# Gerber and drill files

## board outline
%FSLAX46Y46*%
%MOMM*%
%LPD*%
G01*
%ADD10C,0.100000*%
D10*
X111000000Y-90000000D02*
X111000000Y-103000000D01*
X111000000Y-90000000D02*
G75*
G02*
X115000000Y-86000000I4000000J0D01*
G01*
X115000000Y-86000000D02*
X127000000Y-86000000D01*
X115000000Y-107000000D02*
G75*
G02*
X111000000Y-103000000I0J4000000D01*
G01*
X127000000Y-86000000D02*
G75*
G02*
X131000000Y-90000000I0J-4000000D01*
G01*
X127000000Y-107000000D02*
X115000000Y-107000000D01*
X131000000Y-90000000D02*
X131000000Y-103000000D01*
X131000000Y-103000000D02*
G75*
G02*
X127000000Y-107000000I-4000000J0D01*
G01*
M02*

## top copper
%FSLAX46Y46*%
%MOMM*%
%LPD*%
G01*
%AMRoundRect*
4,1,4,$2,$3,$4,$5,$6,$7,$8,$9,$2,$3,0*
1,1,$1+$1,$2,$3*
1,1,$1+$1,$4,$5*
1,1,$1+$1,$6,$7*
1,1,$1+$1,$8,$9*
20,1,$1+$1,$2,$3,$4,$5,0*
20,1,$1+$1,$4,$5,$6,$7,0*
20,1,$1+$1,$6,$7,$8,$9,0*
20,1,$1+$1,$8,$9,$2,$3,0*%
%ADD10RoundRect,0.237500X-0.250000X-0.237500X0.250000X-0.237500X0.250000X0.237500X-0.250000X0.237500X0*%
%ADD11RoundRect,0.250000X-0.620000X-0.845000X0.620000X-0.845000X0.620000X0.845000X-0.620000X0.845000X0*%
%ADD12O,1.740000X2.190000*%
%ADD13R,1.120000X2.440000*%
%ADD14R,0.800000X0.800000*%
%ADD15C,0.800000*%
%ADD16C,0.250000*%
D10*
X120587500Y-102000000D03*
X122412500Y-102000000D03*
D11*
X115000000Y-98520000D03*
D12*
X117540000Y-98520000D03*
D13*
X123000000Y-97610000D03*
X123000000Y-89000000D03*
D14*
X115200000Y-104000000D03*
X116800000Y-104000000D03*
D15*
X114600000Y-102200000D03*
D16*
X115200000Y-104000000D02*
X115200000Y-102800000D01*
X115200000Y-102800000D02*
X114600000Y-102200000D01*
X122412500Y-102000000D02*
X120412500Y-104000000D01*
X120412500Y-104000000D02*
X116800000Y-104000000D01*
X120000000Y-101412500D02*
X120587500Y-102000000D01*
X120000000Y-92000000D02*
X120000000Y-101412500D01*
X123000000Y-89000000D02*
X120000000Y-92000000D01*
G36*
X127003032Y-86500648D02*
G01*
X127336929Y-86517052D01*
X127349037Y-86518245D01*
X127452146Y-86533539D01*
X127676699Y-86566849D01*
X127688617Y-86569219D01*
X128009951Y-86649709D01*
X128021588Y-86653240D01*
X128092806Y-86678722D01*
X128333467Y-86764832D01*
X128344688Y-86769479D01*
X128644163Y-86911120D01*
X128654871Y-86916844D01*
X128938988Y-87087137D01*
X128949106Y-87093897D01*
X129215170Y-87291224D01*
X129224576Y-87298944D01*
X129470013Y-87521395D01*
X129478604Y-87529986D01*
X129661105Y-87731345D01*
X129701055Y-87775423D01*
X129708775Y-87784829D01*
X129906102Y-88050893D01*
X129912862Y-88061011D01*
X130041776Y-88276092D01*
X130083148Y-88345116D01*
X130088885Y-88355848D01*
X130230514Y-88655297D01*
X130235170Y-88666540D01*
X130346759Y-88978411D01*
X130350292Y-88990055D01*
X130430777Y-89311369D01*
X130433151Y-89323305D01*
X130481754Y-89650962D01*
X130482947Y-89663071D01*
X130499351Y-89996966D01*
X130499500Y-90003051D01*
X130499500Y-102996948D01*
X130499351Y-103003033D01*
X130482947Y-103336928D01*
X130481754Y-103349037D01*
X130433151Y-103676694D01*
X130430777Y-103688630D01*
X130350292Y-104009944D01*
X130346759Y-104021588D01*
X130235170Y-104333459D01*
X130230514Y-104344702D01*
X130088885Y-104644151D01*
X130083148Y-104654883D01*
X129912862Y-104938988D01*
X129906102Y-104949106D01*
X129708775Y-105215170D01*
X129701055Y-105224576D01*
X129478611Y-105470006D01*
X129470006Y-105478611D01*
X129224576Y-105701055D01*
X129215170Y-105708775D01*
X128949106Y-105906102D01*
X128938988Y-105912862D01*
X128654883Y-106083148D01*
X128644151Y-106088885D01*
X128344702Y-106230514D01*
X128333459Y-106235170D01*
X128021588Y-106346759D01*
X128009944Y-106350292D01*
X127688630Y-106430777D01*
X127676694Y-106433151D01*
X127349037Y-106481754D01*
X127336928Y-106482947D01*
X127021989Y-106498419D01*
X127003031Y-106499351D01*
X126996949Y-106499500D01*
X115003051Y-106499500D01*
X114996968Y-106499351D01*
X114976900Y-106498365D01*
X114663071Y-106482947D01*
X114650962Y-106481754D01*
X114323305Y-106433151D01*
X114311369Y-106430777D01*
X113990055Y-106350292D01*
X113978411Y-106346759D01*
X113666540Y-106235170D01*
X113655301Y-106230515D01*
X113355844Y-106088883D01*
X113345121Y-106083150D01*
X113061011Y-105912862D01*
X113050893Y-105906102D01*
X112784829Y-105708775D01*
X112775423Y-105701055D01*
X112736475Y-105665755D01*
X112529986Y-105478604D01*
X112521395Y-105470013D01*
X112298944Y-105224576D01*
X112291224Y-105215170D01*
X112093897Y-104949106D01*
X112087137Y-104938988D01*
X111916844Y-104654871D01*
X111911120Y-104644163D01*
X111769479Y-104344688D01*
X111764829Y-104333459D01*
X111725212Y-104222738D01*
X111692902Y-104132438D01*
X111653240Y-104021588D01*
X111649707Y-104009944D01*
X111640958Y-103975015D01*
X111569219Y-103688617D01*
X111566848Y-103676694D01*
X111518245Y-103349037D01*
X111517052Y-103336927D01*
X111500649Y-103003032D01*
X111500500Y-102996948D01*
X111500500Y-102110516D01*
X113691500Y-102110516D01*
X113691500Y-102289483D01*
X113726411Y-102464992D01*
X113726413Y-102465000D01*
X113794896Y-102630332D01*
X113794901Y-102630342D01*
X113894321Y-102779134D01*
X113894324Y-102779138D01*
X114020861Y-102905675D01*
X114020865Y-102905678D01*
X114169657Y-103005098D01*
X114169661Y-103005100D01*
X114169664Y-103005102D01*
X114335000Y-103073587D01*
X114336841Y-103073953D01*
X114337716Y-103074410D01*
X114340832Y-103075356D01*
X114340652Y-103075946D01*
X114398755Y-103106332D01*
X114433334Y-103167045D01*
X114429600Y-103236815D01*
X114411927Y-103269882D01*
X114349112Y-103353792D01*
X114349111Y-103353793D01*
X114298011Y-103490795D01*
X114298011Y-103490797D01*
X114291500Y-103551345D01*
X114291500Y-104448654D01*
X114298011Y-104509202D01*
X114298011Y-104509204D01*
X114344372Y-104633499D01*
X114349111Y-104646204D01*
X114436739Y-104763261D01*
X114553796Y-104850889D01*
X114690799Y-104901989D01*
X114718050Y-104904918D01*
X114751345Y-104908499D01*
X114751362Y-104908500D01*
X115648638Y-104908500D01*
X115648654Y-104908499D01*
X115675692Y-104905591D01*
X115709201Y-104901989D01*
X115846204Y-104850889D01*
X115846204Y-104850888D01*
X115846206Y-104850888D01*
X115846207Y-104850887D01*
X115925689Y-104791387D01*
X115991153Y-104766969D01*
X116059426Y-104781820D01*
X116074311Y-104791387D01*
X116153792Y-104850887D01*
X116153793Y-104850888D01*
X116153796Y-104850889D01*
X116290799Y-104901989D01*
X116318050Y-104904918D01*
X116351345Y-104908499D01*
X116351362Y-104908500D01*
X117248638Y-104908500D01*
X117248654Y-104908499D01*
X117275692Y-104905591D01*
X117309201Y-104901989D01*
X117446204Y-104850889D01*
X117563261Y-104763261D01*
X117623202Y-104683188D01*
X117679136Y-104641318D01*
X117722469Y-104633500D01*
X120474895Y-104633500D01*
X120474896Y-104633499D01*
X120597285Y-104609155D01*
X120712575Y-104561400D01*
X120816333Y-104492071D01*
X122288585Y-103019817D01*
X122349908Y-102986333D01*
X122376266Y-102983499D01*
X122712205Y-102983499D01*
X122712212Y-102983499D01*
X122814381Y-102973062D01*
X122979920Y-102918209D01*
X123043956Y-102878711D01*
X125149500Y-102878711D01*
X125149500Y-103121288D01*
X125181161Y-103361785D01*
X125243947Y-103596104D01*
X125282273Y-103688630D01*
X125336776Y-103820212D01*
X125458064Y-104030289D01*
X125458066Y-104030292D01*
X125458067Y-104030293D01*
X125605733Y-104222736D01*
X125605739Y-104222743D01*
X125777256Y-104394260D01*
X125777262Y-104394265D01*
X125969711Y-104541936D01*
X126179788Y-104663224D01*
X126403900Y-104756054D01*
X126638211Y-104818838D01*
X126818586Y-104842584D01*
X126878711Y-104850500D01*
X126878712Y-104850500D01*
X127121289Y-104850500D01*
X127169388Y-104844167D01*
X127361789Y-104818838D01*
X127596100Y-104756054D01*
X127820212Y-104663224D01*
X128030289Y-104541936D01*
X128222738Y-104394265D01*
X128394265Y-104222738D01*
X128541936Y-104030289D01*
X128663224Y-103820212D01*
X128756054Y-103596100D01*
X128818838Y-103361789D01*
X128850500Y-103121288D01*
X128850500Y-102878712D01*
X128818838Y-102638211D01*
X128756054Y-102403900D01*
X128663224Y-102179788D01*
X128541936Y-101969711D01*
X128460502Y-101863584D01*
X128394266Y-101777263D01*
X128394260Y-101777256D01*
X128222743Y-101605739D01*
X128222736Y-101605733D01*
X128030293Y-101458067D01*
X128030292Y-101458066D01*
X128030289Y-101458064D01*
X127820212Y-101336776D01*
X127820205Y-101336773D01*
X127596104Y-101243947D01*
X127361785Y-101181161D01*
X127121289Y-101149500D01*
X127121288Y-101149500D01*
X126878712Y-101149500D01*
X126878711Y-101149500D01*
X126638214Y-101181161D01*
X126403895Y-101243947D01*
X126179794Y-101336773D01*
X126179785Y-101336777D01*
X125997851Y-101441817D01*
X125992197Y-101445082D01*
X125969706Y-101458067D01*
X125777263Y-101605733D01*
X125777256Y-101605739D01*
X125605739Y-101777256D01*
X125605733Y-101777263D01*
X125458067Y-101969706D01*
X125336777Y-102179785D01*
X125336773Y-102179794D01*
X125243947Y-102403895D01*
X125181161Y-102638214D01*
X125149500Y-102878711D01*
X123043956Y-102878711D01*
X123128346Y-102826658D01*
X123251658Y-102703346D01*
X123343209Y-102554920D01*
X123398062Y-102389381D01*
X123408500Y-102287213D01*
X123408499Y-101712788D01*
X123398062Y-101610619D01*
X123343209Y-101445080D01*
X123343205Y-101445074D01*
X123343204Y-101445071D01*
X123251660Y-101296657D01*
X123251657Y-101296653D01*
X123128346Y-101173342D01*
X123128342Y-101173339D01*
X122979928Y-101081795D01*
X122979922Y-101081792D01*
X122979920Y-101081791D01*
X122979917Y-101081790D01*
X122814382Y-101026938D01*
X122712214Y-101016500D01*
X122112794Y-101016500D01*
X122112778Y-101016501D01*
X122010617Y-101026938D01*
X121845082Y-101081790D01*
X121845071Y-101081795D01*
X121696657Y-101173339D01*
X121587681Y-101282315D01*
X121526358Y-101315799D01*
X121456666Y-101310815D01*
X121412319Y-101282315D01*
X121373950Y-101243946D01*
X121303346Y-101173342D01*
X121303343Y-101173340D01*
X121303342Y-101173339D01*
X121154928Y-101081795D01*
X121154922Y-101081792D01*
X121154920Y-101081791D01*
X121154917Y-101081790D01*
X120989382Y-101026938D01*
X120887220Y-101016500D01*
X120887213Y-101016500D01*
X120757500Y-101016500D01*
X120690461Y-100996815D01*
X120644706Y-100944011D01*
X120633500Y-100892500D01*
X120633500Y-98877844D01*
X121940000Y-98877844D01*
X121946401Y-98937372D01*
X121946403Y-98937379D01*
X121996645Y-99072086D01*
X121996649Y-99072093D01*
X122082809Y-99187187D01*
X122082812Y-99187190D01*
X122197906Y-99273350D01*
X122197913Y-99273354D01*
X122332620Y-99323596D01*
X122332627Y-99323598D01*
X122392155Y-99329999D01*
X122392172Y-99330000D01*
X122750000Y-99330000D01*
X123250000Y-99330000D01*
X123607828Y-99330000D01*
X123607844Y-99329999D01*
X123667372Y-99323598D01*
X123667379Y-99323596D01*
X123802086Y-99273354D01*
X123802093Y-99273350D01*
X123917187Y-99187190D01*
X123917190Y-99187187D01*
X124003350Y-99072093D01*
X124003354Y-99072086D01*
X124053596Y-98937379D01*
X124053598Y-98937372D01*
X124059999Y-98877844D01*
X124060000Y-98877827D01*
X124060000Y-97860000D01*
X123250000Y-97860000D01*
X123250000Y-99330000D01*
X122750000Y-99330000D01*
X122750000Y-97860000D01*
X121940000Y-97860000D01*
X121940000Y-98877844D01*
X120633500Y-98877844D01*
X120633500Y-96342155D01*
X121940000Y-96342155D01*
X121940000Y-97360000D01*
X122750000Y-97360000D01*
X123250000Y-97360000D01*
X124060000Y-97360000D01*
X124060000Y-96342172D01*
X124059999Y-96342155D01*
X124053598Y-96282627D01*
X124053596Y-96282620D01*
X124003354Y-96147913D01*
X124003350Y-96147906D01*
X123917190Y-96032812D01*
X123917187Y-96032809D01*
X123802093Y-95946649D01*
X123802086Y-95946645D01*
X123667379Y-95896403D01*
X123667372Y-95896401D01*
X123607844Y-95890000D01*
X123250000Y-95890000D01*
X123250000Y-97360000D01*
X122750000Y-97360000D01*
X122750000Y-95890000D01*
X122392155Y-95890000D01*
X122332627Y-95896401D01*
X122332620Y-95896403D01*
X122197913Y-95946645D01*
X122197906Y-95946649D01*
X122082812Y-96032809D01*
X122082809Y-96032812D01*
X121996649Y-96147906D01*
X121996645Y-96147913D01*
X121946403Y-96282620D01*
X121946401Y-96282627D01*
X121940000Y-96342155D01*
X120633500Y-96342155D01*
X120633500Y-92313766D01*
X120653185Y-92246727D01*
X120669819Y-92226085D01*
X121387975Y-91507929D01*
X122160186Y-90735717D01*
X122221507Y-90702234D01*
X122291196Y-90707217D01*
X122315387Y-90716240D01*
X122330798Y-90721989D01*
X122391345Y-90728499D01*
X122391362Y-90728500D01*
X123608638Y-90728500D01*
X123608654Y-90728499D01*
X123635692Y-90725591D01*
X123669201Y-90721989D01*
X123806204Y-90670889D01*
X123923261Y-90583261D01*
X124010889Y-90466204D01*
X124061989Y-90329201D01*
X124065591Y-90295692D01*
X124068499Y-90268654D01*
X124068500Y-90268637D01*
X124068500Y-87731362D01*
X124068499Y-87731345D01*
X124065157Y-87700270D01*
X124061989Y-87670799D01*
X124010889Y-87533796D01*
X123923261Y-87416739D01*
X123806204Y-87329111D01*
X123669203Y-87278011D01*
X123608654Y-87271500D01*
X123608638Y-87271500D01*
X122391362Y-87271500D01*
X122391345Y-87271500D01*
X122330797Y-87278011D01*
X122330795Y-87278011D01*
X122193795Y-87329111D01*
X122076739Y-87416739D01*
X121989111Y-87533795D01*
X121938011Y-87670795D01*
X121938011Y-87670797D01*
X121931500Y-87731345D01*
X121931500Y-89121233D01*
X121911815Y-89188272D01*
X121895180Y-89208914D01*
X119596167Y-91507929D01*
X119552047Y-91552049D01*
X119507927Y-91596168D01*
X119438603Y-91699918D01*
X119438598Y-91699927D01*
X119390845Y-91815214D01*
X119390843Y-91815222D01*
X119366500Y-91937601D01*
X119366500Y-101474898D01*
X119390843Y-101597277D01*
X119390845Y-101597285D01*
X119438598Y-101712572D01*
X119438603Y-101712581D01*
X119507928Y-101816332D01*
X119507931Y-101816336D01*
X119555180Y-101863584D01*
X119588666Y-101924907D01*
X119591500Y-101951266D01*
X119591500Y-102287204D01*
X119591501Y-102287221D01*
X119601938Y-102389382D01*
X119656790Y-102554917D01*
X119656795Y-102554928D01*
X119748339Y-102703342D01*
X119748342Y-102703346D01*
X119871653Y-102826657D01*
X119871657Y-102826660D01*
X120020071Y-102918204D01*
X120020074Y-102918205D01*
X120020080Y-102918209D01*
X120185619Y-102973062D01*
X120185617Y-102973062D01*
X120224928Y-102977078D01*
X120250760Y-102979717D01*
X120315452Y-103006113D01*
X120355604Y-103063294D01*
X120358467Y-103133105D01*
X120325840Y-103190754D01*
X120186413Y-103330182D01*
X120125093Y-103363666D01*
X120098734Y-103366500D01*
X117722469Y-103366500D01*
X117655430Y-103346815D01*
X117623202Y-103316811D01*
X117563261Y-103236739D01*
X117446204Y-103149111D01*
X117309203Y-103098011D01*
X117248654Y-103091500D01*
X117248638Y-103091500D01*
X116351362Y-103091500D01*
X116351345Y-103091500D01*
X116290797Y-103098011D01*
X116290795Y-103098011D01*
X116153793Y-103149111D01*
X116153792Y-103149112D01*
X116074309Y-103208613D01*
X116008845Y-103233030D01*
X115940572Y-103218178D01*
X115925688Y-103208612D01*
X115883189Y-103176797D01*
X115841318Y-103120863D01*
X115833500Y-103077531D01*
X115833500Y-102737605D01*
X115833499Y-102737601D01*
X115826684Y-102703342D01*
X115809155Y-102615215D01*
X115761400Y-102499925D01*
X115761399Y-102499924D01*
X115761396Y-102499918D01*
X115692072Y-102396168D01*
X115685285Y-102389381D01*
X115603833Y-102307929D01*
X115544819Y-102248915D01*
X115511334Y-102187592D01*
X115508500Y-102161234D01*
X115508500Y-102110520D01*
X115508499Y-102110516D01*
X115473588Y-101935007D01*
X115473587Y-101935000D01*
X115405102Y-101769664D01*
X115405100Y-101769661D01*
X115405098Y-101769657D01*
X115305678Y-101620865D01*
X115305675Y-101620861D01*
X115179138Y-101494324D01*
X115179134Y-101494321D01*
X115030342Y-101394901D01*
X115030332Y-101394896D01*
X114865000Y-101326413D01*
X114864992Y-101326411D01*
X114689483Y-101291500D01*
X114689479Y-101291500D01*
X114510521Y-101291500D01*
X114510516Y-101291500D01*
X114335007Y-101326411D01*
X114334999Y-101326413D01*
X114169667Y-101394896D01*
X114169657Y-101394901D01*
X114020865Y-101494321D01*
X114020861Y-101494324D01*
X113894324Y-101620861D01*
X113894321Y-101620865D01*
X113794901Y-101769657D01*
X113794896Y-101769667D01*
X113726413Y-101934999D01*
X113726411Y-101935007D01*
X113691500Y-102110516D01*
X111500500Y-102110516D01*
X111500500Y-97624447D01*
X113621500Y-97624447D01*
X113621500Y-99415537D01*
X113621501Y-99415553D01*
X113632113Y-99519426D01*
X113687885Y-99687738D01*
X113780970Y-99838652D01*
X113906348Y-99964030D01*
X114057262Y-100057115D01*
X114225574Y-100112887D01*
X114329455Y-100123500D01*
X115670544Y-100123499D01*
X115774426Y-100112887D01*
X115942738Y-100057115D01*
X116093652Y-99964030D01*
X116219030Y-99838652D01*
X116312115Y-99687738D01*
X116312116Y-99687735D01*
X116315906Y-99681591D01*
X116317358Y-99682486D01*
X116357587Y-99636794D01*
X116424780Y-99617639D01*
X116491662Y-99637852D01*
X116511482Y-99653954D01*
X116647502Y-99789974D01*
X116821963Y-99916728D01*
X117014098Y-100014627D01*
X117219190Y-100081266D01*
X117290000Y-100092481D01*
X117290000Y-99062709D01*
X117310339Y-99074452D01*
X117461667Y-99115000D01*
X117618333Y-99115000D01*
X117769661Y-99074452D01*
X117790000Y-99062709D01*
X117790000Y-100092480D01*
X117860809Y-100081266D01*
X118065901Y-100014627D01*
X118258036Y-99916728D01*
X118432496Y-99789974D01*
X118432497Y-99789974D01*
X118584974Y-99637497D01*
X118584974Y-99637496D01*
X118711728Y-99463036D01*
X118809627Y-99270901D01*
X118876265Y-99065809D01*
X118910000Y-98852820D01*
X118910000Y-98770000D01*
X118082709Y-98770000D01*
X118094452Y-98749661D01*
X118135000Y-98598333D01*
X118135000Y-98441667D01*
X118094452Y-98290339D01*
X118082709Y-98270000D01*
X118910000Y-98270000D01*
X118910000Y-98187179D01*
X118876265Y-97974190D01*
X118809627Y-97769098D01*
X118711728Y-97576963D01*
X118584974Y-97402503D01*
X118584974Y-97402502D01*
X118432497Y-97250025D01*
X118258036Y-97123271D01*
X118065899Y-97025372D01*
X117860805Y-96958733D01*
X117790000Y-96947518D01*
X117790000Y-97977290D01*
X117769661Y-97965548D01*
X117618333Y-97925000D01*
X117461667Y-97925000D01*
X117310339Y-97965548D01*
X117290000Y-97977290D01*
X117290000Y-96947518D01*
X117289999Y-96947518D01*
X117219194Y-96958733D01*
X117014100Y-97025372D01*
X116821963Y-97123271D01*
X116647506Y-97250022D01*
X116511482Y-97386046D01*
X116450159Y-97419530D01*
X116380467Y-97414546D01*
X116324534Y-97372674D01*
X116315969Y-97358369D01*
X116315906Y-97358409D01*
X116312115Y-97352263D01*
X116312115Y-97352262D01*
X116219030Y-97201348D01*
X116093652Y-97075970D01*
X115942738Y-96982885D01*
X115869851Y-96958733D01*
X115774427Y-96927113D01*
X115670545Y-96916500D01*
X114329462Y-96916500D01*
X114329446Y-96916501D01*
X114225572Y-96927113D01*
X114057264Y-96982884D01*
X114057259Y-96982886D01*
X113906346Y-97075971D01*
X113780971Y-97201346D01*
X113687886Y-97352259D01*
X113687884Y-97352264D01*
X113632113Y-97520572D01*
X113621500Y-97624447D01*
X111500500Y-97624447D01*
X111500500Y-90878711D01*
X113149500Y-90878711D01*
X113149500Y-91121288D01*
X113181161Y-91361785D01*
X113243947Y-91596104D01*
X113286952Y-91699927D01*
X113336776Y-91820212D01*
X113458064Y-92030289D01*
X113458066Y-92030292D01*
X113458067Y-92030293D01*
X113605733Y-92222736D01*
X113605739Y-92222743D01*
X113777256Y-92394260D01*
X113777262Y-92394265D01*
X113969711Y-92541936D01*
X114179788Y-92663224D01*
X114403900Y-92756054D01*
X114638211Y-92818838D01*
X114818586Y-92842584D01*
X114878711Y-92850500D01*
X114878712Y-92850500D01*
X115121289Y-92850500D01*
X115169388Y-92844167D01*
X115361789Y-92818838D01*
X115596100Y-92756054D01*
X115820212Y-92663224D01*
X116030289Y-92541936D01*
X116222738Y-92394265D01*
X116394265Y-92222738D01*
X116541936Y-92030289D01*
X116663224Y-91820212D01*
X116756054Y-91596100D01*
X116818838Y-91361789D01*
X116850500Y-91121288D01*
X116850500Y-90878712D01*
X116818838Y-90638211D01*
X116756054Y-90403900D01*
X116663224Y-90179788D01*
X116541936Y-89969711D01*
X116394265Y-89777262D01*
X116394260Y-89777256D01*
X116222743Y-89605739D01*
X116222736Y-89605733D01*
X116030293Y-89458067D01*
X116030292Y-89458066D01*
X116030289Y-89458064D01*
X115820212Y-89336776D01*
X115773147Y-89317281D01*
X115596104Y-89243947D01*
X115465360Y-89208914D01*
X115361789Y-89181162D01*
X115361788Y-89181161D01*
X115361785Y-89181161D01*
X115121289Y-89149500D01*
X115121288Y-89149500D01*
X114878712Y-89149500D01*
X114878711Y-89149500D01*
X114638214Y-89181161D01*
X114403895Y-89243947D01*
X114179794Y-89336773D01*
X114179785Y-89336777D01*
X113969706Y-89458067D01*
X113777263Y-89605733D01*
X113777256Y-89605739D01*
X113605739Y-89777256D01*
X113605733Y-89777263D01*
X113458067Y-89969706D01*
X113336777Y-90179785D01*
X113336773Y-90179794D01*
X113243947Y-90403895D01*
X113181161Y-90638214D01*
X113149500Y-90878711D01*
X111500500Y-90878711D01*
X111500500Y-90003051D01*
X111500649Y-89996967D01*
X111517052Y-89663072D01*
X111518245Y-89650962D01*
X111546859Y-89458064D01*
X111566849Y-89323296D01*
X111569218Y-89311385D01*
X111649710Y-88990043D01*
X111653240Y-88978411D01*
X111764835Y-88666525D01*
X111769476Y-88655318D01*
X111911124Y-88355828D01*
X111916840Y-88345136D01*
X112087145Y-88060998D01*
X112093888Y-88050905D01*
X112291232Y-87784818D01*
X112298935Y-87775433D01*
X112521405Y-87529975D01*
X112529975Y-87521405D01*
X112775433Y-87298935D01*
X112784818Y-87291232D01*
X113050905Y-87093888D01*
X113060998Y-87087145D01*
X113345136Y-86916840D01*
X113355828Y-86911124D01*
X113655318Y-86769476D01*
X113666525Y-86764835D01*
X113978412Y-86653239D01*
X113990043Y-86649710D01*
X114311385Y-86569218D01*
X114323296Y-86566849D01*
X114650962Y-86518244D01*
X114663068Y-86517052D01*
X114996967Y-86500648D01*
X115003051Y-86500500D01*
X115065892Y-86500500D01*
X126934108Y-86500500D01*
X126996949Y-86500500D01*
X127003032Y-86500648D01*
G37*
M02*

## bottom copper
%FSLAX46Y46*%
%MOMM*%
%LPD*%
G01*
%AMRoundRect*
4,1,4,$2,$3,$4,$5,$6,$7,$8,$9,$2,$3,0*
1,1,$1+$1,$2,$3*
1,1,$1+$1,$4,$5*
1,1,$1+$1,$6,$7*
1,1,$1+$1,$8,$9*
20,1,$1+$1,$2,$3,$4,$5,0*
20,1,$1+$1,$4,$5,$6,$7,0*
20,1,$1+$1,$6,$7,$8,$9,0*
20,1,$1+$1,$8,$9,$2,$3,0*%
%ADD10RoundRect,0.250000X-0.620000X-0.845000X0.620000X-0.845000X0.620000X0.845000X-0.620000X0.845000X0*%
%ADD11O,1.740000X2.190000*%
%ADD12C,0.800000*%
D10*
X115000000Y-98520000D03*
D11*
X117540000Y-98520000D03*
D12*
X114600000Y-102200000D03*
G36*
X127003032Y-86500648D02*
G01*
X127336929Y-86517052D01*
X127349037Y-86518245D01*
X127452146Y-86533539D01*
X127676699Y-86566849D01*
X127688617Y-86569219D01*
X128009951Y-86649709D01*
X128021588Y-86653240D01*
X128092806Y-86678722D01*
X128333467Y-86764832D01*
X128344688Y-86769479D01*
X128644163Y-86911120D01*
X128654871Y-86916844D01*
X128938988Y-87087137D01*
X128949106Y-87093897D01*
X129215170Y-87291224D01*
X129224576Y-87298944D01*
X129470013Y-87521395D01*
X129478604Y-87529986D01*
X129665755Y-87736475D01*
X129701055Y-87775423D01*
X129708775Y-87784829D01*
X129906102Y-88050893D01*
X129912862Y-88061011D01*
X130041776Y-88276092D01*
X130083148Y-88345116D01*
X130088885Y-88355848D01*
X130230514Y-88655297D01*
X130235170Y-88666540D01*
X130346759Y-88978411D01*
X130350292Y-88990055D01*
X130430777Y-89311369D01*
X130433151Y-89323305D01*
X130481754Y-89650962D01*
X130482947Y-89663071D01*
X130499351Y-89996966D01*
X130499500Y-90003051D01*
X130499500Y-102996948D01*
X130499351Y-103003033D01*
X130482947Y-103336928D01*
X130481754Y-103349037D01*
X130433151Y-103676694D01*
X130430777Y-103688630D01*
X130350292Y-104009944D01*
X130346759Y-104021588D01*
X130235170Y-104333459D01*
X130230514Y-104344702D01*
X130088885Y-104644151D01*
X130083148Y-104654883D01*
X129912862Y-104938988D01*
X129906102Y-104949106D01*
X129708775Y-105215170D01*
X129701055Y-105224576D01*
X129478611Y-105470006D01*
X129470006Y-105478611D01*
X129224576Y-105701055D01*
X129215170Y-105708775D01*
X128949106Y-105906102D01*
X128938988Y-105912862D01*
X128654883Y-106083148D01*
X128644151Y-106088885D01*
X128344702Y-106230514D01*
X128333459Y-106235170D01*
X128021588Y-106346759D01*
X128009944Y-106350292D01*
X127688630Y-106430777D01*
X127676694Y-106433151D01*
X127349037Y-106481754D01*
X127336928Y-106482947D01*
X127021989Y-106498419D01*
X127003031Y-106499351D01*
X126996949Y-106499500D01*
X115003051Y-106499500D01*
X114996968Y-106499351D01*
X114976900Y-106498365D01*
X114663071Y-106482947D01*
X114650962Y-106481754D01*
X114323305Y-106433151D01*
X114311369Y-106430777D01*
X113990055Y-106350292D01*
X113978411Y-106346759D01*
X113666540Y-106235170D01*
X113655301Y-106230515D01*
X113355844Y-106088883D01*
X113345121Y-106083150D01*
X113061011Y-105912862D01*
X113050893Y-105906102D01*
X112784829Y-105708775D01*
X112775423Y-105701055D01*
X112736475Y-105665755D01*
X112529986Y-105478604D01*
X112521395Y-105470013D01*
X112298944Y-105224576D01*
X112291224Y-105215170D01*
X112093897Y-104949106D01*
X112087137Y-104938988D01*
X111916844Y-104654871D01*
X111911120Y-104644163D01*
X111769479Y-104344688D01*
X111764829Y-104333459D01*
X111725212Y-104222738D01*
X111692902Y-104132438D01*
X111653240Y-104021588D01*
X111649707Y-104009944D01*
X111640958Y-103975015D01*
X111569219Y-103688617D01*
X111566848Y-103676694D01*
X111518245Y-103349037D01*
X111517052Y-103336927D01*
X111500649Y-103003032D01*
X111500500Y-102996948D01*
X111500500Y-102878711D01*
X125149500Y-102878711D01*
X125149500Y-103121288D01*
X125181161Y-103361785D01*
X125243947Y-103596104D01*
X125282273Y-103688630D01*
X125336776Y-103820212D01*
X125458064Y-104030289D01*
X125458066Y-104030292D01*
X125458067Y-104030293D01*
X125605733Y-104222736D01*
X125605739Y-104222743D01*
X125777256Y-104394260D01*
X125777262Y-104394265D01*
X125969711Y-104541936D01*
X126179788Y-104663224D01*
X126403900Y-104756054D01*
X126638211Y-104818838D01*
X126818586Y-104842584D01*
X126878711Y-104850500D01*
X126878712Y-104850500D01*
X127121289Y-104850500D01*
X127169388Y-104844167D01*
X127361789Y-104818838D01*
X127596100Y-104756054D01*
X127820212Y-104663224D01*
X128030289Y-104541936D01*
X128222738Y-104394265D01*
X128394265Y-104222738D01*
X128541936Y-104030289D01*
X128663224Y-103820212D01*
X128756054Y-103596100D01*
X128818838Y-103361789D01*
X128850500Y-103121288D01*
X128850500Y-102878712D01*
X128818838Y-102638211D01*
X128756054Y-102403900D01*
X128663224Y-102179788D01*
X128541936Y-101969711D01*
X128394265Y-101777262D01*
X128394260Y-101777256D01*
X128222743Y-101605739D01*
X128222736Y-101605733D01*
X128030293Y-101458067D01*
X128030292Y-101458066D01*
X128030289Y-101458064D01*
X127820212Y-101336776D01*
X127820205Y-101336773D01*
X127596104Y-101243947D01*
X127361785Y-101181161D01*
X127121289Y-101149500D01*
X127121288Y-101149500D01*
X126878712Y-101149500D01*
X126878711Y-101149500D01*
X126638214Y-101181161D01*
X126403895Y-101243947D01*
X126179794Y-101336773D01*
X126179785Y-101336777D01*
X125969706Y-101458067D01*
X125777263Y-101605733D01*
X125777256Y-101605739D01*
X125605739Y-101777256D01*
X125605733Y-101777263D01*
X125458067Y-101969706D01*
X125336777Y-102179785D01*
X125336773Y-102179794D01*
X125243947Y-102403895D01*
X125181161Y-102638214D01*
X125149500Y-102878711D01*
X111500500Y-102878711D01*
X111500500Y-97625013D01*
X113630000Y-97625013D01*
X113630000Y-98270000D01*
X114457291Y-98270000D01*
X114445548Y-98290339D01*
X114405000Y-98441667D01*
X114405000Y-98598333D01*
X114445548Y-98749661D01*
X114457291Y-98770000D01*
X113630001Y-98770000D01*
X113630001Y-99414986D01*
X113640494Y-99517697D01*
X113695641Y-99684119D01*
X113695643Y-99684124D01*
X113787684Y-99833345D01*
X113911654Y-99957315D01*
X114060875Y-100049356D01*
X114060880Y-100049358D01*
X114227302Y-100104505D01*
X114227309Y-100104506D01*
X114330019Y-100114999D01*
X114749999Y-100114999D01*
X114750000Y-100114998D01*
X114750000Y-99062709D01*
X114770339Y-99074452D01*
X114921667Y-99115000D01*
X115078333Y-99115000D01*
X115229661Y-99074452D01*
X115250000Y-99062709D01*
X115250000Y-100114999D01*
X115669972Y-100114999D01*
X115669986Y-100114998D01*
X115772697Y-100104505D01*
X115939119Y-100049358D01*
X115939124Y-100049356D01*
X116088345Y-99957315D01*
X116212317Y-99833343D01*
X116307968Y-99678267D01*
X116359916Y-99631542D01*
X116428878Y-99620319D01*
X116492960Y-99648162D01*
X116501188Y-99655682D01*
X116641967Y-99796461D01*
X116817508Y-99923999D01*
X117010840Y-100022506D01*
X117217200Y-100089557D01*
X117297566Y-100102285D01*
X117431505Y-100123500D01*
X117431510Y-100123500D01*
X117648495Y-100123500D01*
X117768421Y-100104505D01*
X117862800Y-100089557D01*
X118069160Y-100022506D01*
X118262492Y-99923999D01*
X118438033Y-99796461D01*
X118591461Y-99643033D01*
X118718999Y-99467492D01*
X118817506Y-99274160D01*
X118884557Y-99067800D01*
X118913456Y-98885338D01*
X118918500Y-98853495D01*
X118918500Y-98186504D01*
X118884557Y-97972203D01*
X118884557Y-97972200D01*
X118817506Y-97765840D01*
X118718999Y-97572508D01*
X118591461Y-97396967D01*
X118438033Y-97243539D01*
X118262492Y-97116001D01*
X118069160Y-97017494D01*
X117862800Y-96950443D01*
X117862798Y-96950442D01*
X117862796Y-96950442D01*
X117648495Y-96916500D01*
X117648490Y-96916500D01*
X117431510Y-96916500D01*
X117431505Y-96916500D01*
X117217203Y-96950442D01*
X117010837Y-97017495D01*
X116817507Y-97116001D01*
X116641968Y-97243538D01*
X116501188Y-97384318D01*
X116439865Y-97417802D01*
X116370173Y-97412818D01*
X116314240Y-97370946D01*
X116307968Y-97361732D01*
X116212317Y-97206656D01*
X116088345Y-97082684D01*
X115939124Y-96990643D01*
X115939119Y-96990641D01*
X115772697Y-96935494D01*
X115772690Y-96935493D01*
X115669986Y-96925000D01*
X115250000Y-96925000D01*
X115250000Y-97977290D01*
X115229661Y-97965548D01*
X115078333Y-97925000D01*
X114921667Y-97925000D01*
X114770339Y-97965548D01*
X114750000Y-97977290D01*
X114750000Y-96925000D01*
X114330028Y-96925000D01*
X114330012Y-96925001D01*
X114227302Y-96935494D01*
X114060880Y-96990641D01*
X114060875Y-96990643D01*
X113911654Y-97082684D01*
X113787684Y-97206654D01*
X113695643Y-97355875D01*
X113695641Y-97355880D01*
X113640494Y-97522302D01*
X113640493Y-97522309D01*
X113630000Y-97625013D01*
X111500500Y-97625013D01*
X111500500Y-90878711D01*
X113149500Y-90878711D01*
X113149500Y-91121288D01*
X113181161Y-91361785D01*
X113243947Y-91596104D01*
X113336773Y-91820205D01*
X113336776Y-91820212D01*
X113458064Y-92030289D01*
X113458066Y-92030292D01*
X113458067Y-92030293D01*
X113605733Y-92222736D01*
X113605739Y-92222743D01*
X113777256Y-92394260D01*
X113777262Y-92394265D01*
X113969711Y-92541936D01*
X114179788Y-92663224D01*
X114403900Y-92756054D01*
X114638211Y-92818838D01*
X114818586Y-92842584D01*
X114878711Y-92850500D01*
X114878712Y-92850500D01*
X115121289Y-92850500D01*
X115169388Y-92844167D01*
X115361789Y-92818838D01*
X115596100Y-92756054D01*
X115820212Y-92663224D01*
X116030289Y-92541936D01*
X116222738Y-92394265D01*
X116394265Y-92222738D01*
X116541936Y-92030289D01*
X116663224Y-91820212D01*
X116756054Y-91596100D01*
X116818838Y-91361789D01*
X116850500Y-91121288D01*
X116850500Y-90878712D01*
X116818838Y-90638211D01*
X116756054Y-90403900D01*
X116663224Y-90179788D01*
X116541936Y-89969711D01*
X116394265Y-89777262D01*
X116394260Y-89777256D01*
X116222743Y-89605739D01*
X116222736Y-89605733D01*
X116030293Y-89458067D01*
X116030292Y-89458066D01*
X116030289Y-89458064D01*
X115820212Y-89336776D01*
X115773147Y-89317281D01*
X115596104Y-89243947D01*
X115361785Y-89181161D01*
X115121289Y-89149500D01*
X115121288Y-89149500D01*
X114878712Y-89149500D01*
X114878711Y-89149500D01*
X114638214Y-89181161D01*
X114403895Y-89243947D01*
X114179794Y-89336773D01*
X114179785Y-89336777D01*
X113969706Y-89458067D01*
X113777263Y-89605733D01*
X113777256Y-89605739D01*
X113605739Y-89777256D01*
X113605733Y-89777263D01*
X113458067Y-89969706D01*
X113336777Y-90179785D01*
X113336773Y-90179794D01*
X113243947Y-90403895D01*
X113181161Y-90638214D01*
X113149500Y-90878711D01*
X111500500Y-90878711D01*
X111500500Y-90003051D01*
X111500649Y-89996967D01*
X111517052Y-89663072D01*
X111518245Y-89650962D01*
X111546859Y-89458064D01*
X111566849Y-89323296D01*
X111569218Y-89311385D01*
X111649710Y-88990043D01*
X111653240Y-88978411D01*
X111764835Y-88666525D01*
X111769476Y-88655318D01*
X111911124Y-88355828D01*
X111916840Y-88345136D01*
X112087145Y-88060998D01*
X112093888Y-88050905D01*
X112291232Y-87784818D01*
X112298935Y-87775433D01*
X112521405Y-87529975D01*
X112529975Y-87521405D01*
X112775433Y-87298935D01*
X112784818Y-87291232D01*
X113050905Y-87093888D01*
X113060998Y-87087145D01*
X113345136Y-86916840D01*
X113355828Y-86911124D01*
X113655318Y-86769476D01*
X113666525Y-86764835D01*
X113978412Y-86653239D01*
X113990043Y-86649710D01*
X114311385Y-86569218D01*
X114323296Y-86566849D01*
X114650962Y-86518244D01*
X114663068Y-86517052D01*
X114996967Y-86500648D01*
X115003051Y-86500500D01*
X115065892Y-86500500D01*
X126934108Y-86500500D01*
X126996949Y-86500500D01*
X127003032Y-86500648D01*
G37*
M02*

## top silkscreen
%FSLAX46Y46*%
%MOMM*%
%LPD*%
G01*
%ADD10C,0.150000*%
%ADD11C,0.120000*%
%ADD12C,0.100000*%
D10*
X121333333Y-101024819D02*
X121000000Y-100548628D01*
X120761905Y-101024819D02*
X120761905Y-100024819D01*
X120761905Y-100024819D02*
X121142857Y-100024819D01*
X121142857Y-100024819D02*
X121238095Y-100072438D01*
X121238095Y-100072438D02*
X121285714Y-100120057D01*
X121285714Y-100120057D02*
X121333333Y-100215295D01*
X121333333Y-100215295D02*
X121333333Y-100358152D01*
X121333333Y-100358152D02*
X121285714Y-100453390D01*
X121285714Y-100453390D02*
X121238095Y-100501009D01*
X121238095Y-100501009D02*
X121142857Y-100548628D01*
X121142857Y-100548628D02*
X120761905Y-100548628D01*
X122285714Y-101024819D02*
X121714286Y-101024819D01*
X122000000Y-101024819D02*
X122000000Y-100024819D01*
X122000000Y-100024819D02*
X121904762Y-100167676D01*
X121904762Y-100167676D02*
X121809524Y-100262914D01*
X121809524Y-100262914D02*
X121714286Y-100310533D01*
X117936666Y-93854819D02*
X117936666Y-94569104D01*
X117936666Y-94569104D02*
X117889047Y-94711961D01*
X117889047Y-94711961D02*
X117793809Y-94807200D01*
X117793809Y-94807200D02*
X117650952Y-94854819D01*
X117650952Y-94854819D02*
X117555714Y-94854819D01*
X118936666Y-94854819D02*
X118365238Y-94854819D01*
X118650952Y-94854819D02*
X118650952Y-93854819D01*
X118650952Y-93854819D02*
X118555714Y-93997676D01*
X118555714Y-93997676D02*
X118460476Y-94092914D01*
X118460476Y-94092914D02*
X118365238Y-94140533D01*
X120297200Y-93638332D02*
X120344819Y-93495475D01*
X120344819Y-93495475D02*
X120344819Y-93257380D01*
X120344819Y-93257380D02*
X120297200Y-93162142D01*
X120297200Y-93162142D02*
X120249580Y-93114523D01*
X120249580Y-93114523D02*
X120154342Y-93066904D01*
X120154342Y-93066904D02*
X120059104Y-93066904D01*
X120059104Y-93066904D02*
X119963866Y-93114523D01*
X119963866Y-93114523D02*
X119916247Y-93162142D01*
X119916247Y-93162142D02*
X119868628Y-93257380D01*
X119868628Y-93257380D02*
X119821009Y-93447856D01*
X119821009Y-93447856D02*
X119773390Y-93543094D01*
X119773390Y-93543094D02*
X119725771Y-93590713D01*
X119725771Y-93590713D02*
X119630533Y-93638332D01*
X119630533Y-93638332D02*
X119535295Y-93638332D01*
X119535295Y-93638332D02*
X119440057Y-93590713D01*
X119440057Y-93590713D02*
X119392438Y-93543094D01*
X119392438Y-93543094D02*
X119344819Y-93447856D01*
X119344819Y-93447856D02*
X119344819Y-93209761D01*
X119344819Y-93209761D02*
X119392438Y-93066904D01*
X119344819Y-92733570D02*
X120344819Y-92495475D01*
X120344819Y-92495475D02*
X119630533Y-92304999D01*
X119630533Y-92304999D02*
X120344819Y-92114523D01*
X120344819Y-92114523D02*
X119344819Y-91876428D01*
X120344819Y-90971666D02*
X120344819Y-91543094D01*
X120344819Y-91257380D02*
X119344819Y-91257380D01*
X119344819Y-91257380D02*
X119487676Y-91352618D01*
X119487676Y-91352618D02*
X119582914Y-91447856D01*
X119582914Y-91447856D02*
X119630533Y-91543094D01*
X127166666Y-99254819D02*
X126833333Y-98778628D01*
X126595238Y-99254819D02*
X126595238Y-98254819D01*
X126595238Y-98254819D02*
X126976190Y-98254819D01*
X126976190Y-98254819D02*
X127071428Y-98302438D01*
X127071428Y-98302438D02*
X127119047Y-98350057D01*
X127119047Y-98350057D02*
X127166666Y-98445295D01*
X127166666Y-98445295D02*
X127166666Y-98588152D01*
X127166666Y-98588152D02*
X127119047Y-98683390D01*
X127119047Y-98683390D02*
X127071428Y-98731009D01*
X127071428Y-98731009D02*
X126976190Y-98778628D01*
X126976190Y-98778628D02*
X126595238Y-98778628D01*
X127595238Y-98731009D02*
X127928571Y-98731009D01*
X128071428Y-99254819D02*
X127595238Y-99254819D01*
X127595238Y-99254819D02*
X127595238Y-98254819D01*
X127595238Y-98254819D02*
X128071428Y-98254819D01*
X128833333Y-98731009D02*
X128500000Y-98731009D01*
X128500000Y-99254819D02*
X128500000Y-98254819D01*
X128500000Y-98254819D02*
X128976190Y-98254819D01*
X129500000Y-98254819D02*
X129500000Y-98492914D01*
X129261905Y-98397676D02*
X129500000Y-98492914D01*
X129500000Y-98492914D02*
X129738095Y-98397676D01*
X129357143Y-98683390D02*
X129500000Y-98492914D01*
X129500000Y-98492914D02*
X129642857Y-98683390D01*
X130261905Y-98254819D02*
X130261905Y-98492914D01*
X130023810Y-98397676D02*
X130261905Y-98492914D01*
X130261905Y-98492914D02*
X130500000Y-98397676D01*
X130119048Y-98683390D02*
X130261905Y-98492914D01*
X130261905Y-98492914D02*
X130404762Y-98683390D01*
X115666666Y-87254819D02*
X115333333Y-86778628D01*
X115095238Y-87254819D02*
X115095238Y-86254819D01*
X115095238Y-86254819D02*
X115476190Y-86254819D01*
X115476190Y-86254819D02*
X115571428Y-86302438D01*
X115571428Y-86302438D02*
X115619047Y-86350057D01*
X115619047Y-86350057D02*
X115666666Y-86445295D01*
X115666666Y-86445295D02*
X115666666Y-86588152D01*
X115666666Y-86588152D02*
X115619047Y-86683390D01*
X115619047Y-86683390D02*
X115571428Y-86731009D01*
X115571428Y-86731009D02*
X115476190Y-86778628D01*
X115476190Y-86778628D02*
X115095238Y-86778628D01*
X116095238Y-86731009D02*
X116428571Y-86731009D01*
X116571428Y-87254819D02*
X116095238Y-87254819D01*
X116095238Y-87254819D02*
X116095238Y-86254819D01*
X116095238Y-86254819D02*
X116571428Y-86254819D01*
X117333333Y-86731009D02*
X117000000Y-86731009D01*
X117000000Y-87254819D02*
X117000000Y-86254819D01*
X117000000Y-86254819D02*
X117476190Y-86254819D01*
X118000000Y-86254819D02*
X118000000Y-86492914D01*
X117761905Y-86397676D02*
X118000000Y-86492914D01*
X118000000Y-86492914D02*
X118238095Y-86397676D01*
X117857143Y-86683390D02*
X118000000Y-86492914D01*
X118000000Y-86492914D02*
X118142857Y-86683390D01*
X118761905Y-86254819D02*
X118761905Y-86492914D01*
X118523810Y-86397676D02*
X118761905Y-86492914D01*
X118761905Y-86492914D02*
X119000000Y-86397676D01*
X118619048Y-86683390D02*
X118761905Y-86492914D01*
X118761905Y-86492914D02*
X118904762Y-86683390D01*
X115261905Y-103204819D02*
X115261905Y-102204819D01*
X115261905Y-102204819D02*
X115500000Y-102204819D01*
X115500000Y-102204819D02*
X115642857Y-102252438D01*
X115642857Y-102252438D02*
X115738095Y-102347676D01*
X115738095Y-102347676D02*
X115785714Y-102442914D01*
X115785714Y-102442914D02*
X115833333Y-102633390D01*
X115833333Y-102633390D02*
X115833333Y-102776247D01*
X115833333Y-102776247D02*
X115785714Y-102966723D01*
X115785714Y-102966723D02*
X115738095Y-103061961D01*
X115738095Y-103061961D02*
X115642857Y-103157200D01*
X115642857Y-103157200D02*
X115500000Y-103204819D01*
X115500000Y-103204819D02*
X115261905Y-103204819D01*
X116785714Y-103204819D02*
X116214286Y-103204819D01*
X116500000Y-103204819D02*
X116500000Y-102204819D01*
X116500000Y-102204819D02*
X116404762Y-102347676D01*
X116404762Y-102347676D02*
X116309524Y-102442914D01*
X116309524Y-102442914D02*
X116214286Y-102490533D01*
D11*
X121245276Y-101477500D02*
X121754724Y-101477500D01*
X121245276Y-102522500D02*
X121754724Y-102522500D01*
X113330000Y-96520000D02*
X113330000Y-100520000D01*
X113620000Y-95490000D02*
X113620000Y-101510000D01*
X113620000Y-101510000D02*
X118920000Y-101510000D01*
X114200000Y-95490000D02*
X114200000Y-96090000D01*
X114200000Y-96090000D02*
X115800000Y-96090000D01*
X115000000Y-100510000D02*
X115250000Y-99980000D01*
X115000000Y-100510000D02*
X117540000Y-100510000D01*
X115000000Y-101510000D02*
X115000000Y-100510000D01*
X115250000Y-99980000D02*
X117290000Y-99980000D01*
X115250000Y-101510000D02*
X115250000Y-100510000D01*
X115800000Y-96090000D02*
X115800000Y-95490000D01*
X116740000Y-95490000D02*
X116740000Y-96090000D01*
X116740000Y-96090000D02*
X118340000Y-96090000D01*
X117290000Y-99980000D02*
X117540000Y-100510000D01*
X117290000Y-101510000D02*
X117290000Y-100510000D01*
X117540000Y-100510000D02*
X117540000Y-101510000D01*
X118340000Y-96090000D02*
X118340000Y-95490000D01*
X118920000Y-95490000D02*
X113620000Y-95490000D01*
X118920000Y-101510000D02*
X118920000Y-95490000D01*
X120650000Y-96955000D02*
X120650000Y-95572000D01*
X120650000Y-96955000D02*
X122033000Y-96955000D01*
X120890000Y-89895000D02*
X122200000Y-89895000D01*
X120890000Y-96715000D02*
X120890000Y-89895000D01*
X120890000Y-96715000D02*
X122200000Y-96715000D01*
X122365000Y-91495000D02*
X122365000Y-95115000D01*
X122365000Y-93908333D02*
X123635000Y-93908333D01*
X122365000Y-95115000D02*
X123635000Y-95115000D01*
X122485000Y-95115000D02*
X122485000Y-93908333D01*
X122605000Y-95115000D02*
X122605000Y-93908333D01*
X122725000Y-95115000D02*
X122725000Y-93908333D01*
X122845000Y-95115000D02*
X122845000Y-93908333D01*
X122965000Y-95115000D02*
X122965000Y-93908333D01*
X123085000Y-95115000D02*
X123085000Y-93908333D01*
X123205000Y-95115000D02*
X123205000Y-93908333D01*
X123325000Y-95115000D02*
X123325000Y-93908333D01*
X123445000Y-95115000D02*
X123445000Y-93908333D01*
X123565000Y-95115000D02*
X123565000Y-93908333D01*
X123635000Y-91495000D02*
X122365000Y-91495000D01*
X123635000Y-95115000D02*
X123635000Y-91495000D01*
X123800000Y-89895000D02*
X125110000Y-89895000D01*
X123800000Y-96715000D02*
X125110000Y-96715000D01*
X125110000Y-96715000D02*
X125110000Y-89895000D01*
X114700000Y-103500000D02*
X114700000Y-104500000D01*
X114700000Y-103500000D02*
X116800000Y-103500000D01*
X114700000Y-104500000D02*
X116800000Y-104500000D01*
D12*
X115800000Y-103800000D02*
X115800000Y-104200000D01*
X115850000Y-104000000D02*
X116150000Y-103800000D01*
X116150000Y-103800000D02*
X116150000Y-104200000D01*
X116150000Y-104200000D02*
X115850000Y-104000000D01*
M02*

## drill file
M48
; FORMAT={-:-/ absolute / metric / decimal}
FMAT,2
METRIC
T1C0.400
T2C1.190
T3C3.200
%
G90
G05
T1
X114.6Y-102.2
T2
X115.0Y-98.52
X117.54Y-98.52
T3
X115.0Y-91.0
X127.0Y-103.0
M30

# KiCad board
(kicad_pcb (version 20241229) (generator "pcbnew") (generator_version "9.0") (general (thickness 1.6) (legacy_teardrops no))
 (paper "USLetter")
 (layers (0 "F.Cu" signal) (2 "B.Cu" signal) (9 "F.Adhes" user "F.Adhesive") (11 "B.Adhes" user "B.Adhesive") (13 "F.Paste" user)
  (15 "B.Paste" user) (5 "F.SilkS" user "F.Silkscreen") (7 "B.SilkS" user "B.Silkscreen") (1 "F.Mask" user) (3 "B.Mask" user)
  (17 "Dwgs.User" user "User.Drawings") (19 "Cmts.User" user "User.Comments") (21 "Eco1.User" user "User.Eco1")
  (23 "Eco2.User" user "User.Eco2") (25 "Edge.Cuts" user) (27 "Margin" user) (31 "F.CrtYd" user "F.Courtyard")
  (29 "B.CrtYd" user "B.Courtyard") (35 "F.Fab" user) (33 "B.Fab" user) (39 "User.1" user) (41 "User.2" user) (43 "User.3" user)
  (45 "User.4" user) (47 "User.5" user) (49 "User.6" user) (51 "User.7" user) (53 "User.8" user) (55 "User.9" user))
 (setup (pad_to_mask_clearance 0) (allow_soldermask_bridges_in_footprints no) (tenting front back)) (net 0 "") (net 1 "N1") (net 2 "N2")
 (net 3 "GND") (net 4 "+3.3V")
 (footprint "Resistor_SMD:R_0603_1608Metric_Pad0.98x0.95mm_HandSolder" (layer "F.Cu") (at 121.5 102)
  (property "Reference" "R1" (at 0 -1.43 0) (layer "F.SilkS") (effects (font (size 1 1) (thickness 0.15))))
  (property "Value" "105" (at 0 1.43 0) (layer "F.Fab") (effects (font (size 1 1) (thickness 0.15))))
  (fp_line (start -0.254724 -0.5225) (end 0.254724 -0.5225) (stroke (width 0.12) (type solid)) (layer "F.SilkS"))
  (fp_line (start -0.254724 0.5225) (end 0.254724 0.5225) (stroke (width 0.12) (type solid)) (layer "F.SilkS"))
  (pad "1" smd roundrect (at -0.9125 0) (size 0.975 0.95) (layers "F.Cu" "F.Mask" "F.Paste") (roundrect_rratio 0.25) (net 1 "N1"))
  (pad "2" smd roundrect (at 0.9125 0) (size 0.975 0.95) (layers "F.Cu" "F.Mask" "F.Paste") (roundrect_rratio 0.25) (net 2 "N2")))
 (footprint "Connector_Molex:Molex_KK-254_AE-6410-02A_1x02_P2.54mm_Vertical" (layer "F.Cu") (at 115 98.52)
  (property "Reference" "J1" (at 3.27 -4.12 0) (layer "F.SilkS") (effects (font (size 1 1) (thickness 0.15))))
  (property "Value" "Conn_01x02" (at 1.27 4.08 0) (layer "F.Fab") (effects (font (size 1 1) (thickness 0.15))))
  (fp_line (start -1.67 -2) (end -1.67 2) (stroke (width 0.12) (type solid)) (layer "F.SilkS"))
  (fp_line (start -1.38 -3.03) (end -1.38 2.99) (stroke (width 0.12) (type solid)) (layer "F.SilkS"))
  (fp_line (start -1.38 2.99) (end 3.92 2.99) (stroke (width 0.12) (type solid)) (layer "F.SilkS"))
  (fp_line (start -0.8 -3.03) (end -0.8 -2.43) (stroke (width 0.12) (type solid)) (layer "F.SilkS"))
  (fp_line (start -0.8 -2.43) (end 0.8 -2.43) (stroke (width 0.12) (type solid)) (layer "F.SilkS"))
  (fp_line (start 0 1.99) (end 0.25 1.46) (stroke (width 0.12) (type solid)) (layer "F.SilkS"))
  (fp_line (start 0 1.99) (end 2.54 1.99) (stroke (width 0.12) (type solid)) (layer "F.SilkS"))
  (fp_line (start 0 2.99) (end 0 1.99) (stroke (width 0.12) (type solid)) (layer "F.SilkS"))
  (fp_line (start 0.25 1.46) (end 2.29 1.46) (stroke (width 0.12) (type solid)) (layer "F.SilkS"))
  (fp_line (start 0.25 2.99) (end 0.25 1.99) (stroke (width 0.12) (type solid)) (layer "F.SilkS"))
  (fp_line (start 0.8 -2.43) (end 0.8 -3.03) (stroke (width 0.12) (type solid)) (layer "F.SilkS"))
  (fp_line (start 1.74 -3.03) (end 1.74 -2.43) (stroke (width 0.12) (type solid)) (layer "F.SilkS"))
  (fp_line (start 1.74 -2.43) (end 3.34 -2.43) (stroke (width 0.12) (type solid)) (layer "F.SilkS"))
  (fp_line (start 2.29 1.46) (end 2.54 1.99) (stroke (width 0.12) (type solid)) (layer "F.SilkS"))
  (fp_line (start 2.29 2.99) (end 2.29 1.99) (stroke (width 0.12) (type solid)) (layer "F.SilkS"))
  (fp_line (start 2.54 1.99) (end 2.54 2.99) (stroke (width 0.12) (type solid)) (layer "F.SilkS"))
  (fp_line (start 3.34 -2.43) (end 3.34 -3.03) (stroke (width 0.12) (type solid)) (layer "F.SilkS"))
  (fp_line (start 3.92 -3.03) (end -1.38 -3.03) (stroke (width 0.12) (type solid)) (layer "F.SilkS"))
  (fp_line (start 3.92 2.99) (end 3.92 -3.03) (stroke (width 0.12) (type solid)) (layer "F.SilkS"))
  (pad "1" thru_hole roundrect (at 0 0) (size 1.74 2.19) (drill 1.19) (layers "*.Cu" "*.Mask") (remove_unused_layers no)
   (roundrect_rratio 0.143678) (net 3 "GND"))
  (pad "2" thru_hole oval (at 2.54 0) (size 1.74 2.19) (drill 1.19) (layers "*.Cu" "*.Mask") (remove_unused_layers no) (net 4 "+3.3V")))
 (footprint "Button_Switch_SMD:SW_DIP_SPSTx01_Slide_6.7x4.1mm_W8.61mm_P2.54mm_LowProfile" (layer "F.Cu") (at 123 93.305 90)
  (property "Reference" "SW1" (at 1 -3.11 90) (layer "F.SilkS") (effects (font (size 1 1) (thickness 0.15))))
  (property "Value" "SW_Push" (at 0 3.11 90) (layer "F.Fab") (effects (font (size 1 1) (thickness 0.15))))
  (fp_line (start -3.65 -2.35) (end -2.267 -2.35) (stroke (width 0.12) (type solid)) (layer "F.SilkS"))
  (fp_line (start -3.65 -2.35) (end -3.65 -0.967) (stroke (width 0.12) (type solid)) (layer "F.SilkS"))
  (fp_line (start 3.41 -2.11) (end 3.41 -0.8) (stroke (width 0.12) (type solid)) (layer "F.SilkS"))
  (fp_line (start -3.41 -2.11) (end 3.41 -2.11) (stroke (width 0.12) (type solid)) (layer "F.SilkS"))
  (fp_line (start -3.41 -2.11) (end -3.41 -0.8) (stroke (width 0.12) (type solid)) (layer "F.SilkS"))
  (fp_line (start 1.81 -0.635) (end -1.81 -0.635) (stroke (width 0.12) (type solid)) (layer "F.SilkS"))
  (fp_line (start -0.603333 -0.635) (end -0.603333 0.635) (stroke (width 0.12) (type solid)) (layer "F.SilkS"))
  (fp_line (start -1.81 -0.635) (end -1.81 0.635) (stroke (width 0.12) (type solid)) (layer "F.SilkS"))
  (fp_line (start -1.81 -0.515) (end -0.603333 -0.515) (stroke (width 0.12) (type solid)) (layer "F.SilkS"))
  (fp_line (start -1.81 -0.395) (end -0.603333 -0.395) (stroke (width 0.12) (type solid)) (layer "F.SilkS"))
  (fp_line (start -1.81 -0.275) (end -0.603333 -0.275) (stroke (width 0.12) (type solid)) (layer "F.SilkS"))
  (fp_line (start -1.81 -0.155) (end -0.603333 -0.155) (stroke (width 0.12) (type solid)) (layer "F.SilkS"))
  (fp_line (start -1.81 -0.035) (end -0.603333 -0.035) (stroke (width 0.12) (type solid)) (layer "F.SilkS"))
  (fp_line (start -1.81 0.085) (end -0.603333 0.085) (stroke (width 0.12) (type solid)) (layer "F.SilkS"))
  (fp_line (start -1.81 0.205) (end -0.603333 0.205) (stroke (width 0.12) (type solid)) (layer "F.SilkS"))
  (fp_line (start -1.81 0.325) (end -0.603333 0.325) (stroke (width 0.12) (type solid)) (layer "F.SilkS"))
  (fp_line (start -1.81 0.445) (end -0.603333 0.445) (stroke (width 0.12) (type solid)) (layer "F.SilkS"))
  (fp_line (start -1.81 0.565) (end -0.603333 0.565) (stroke (width 0.12) (type solid)) (layer "F.SilkS"))
  (fp_line (start 1.81 0.635) (end 1.81 -0.635) (stroke (width 0.12) (type solid)) (layer "F.SilkS"))
  (fp_line (start -1.81 0.635) (end 1.81 0.635) (stroke (width 0.12) (type solid)) (layer "F.SilkS"))
  (fp_line (start 3.41 0.8) (end 3.41 2.11) (stroke (width 0.12) (type solid)) (layer "F.SilkS"))
  (fp_line (start -3.41 0.8) (end -3.41 2.11) (stroke (width 0.12) (type solid)) (layer "F.SilkS"))
  (fp_line (start -3.41 2.11) (end 3.41 2.11) (stroke (width 0.12) (type solid)) (layer "F.SilkS"))
  (pad "1" smd rect (at -4.305 0 90) (size 2.44 1.12) (layers "F.Cu" "F.Mask" "F.Paste") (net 4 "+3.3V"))
  (pad "2" smd rect (at 4.305 0 90) (size 2.44 1.12) (layers "F.Cu" "F.Mask" "F.Paste") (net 1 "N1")))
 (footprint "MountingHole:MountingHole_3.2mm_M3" (layer "F.Cu") (at 127 103)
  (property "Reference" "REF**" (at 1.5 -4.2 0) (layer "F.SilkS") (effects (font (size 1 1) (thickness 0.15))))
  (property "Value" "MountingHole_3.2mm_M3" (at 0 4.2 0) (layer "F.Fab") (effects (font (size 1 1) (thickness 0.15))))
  (pad "" np_thru_hole circle (at 0 0) (size 3.2 3.2) (drill 3.2) (layers "*.Cu" "*.Mask")))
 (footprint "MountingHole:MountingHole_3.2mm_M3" (layer "F.Cu") (at 115 91)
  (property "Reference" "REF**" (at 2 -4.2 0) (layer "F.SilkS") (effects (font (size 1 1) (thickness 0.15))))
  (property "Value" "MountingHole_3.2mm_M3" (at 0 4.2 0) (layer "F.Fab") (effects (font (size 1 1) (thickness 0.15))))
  (pad "" np_thru_hole circle (at 0 0) (size 3.2 3.2) (drill 3.2) (layers "*.Cu" "*.Mask")))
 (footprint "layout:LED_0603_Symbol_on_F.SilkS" (layer "F.Cu") (at 116 104)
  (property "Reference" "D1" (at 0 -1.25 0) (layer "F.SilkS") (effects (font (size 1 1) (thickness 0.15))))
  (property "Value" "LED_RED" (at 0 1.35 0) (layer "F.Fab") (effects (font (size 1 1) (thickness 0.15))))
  (fp_line (start -1.3 -0.5) (end -1.3 0.5) (stroke (width 0.12) (type solid)) (layer "F.SilkS"))
  (fp_line (start -1.3 -0.5) (end 0.8 -0.5) (stroke (width 0.12) (type solid)) (layer "F.SilkS"))
  (fp_line (start -1.3 0.5) (end 0.8 0.5) (stroke (width 0.12) (type solid)) (layer "F.SilkS"))
  (fp_line (start -0.2 -0.2) (end -0.2 0.2) (stroke (width 0.1) (type solid)) (layer "F.SilkS"))
  (fp_line (start -0.15 0) (end 0.15 -0.2) (stroke (width 0.1) (type solid)) (layer "F.SilkS"))
  (fp_line (start 0.15 -0.2) (end 0.15 0.2) (stroke (width 0.1) (type solid)) (layer "F.SilkS"))
  (fp_line (start 0.15 0.2) (end -0.15 0) (stroke (width 0.1) (type solid)) (layer "F.SilkS"))
  (pad "1" smd rect (at -0.8 0 180) (size 0.8 0.8) (layers "F.Cu" "F.Mask" "F.Paste") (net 3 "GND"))
  (pad "2" smd rect (at 0.8 0 180) (size 0.8 0.8) (layers "F.Cu" "F.Mask" "F.Paste") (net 2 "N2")))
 (gr_line (start 111 90) (end 111 103) (stroke (width 0.1) (type default)) (layer "Edge.Cuts"))
 (gr_arc (start 111 90) (mid 112.171573 87.171573) (end 115 86) (stroke (width 0.1) (type default)) (layer "Edge.Cuts"))
 (gr_line (start 115 86) (end 127 86) (stroke (width 0.1) (type default)) (layer "Edge.Cuts"))
 (gr_arc (start 115 107) (mid 112.171573 105.828427) (end 111 103) (stroke (width 0.1) (type default)) (layer "Edge.Cuts"))
 (gr_arc (start 127 86) (mid 129.828427 87.171573) (end 131 90) (stroke (width 0.1) (type default)) (layer "Edge.Cuts"))
 (gr_line (start 127 107) (end 115 107) (stroke (width 0.1) (type default)) (layer "Edge.Cuts"))
 (gr_line (start 131 90) (end 131 103) (stroke (width 0.1) (type default)) (layer "Edge.Cuts"))
 (gr_arc (start 131 103) (mid 129.828427 105.828427) (end 127 107) (stroke (width 0.1) (type default)) (layer "Edge.Cuts"))
 (segment (start 115.2 104) (end 115.2 102.8) (width 0.25) (layer "F.Cu") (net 3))
 (segment (start 115.2 102.8) (end 114.6 102.2) (width 0.25) (layer "F.Cu") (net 3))
 (via (at 114.6 102.2) (size 0.8) (drill 0.4) (layers "F.Cu" "B.Cu") (free yes) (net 3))
 (segment (start 122.4125 102) (end 120.4125 104) (width 0.25) (layer "F.Cu") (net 2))
 (segment (start 120.4125 104) (end 116.8 104) (width 0.25) (layer "F.Cu") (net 2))
 (segment (start 120 101.4125) (end 120.5875 102) (width 0.25) (layer "F.Cu") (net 1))
 (segment (start 120 92) (end 120 101.4125) (width 0.25) (layer "F.Cu") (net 1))
 (segment (start 123 89) (end 120 92) (width 0.25) (layer "F.Cu") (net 1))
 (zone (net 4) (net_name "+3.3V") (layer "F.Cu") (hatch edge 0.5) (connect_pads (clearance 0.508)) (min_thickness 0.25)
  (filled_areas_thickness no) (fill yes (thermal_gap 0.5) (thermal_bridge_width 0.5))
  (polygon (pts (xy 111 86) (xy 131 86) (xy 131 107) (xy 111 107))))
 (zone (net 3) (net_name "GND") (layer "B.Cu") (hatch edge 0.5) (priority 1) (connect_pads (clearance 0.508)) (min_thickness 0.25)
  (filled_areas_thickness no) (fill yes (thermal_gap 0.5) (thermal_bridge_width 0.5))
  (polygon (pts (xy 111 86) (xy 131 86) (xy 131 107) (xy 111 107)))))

